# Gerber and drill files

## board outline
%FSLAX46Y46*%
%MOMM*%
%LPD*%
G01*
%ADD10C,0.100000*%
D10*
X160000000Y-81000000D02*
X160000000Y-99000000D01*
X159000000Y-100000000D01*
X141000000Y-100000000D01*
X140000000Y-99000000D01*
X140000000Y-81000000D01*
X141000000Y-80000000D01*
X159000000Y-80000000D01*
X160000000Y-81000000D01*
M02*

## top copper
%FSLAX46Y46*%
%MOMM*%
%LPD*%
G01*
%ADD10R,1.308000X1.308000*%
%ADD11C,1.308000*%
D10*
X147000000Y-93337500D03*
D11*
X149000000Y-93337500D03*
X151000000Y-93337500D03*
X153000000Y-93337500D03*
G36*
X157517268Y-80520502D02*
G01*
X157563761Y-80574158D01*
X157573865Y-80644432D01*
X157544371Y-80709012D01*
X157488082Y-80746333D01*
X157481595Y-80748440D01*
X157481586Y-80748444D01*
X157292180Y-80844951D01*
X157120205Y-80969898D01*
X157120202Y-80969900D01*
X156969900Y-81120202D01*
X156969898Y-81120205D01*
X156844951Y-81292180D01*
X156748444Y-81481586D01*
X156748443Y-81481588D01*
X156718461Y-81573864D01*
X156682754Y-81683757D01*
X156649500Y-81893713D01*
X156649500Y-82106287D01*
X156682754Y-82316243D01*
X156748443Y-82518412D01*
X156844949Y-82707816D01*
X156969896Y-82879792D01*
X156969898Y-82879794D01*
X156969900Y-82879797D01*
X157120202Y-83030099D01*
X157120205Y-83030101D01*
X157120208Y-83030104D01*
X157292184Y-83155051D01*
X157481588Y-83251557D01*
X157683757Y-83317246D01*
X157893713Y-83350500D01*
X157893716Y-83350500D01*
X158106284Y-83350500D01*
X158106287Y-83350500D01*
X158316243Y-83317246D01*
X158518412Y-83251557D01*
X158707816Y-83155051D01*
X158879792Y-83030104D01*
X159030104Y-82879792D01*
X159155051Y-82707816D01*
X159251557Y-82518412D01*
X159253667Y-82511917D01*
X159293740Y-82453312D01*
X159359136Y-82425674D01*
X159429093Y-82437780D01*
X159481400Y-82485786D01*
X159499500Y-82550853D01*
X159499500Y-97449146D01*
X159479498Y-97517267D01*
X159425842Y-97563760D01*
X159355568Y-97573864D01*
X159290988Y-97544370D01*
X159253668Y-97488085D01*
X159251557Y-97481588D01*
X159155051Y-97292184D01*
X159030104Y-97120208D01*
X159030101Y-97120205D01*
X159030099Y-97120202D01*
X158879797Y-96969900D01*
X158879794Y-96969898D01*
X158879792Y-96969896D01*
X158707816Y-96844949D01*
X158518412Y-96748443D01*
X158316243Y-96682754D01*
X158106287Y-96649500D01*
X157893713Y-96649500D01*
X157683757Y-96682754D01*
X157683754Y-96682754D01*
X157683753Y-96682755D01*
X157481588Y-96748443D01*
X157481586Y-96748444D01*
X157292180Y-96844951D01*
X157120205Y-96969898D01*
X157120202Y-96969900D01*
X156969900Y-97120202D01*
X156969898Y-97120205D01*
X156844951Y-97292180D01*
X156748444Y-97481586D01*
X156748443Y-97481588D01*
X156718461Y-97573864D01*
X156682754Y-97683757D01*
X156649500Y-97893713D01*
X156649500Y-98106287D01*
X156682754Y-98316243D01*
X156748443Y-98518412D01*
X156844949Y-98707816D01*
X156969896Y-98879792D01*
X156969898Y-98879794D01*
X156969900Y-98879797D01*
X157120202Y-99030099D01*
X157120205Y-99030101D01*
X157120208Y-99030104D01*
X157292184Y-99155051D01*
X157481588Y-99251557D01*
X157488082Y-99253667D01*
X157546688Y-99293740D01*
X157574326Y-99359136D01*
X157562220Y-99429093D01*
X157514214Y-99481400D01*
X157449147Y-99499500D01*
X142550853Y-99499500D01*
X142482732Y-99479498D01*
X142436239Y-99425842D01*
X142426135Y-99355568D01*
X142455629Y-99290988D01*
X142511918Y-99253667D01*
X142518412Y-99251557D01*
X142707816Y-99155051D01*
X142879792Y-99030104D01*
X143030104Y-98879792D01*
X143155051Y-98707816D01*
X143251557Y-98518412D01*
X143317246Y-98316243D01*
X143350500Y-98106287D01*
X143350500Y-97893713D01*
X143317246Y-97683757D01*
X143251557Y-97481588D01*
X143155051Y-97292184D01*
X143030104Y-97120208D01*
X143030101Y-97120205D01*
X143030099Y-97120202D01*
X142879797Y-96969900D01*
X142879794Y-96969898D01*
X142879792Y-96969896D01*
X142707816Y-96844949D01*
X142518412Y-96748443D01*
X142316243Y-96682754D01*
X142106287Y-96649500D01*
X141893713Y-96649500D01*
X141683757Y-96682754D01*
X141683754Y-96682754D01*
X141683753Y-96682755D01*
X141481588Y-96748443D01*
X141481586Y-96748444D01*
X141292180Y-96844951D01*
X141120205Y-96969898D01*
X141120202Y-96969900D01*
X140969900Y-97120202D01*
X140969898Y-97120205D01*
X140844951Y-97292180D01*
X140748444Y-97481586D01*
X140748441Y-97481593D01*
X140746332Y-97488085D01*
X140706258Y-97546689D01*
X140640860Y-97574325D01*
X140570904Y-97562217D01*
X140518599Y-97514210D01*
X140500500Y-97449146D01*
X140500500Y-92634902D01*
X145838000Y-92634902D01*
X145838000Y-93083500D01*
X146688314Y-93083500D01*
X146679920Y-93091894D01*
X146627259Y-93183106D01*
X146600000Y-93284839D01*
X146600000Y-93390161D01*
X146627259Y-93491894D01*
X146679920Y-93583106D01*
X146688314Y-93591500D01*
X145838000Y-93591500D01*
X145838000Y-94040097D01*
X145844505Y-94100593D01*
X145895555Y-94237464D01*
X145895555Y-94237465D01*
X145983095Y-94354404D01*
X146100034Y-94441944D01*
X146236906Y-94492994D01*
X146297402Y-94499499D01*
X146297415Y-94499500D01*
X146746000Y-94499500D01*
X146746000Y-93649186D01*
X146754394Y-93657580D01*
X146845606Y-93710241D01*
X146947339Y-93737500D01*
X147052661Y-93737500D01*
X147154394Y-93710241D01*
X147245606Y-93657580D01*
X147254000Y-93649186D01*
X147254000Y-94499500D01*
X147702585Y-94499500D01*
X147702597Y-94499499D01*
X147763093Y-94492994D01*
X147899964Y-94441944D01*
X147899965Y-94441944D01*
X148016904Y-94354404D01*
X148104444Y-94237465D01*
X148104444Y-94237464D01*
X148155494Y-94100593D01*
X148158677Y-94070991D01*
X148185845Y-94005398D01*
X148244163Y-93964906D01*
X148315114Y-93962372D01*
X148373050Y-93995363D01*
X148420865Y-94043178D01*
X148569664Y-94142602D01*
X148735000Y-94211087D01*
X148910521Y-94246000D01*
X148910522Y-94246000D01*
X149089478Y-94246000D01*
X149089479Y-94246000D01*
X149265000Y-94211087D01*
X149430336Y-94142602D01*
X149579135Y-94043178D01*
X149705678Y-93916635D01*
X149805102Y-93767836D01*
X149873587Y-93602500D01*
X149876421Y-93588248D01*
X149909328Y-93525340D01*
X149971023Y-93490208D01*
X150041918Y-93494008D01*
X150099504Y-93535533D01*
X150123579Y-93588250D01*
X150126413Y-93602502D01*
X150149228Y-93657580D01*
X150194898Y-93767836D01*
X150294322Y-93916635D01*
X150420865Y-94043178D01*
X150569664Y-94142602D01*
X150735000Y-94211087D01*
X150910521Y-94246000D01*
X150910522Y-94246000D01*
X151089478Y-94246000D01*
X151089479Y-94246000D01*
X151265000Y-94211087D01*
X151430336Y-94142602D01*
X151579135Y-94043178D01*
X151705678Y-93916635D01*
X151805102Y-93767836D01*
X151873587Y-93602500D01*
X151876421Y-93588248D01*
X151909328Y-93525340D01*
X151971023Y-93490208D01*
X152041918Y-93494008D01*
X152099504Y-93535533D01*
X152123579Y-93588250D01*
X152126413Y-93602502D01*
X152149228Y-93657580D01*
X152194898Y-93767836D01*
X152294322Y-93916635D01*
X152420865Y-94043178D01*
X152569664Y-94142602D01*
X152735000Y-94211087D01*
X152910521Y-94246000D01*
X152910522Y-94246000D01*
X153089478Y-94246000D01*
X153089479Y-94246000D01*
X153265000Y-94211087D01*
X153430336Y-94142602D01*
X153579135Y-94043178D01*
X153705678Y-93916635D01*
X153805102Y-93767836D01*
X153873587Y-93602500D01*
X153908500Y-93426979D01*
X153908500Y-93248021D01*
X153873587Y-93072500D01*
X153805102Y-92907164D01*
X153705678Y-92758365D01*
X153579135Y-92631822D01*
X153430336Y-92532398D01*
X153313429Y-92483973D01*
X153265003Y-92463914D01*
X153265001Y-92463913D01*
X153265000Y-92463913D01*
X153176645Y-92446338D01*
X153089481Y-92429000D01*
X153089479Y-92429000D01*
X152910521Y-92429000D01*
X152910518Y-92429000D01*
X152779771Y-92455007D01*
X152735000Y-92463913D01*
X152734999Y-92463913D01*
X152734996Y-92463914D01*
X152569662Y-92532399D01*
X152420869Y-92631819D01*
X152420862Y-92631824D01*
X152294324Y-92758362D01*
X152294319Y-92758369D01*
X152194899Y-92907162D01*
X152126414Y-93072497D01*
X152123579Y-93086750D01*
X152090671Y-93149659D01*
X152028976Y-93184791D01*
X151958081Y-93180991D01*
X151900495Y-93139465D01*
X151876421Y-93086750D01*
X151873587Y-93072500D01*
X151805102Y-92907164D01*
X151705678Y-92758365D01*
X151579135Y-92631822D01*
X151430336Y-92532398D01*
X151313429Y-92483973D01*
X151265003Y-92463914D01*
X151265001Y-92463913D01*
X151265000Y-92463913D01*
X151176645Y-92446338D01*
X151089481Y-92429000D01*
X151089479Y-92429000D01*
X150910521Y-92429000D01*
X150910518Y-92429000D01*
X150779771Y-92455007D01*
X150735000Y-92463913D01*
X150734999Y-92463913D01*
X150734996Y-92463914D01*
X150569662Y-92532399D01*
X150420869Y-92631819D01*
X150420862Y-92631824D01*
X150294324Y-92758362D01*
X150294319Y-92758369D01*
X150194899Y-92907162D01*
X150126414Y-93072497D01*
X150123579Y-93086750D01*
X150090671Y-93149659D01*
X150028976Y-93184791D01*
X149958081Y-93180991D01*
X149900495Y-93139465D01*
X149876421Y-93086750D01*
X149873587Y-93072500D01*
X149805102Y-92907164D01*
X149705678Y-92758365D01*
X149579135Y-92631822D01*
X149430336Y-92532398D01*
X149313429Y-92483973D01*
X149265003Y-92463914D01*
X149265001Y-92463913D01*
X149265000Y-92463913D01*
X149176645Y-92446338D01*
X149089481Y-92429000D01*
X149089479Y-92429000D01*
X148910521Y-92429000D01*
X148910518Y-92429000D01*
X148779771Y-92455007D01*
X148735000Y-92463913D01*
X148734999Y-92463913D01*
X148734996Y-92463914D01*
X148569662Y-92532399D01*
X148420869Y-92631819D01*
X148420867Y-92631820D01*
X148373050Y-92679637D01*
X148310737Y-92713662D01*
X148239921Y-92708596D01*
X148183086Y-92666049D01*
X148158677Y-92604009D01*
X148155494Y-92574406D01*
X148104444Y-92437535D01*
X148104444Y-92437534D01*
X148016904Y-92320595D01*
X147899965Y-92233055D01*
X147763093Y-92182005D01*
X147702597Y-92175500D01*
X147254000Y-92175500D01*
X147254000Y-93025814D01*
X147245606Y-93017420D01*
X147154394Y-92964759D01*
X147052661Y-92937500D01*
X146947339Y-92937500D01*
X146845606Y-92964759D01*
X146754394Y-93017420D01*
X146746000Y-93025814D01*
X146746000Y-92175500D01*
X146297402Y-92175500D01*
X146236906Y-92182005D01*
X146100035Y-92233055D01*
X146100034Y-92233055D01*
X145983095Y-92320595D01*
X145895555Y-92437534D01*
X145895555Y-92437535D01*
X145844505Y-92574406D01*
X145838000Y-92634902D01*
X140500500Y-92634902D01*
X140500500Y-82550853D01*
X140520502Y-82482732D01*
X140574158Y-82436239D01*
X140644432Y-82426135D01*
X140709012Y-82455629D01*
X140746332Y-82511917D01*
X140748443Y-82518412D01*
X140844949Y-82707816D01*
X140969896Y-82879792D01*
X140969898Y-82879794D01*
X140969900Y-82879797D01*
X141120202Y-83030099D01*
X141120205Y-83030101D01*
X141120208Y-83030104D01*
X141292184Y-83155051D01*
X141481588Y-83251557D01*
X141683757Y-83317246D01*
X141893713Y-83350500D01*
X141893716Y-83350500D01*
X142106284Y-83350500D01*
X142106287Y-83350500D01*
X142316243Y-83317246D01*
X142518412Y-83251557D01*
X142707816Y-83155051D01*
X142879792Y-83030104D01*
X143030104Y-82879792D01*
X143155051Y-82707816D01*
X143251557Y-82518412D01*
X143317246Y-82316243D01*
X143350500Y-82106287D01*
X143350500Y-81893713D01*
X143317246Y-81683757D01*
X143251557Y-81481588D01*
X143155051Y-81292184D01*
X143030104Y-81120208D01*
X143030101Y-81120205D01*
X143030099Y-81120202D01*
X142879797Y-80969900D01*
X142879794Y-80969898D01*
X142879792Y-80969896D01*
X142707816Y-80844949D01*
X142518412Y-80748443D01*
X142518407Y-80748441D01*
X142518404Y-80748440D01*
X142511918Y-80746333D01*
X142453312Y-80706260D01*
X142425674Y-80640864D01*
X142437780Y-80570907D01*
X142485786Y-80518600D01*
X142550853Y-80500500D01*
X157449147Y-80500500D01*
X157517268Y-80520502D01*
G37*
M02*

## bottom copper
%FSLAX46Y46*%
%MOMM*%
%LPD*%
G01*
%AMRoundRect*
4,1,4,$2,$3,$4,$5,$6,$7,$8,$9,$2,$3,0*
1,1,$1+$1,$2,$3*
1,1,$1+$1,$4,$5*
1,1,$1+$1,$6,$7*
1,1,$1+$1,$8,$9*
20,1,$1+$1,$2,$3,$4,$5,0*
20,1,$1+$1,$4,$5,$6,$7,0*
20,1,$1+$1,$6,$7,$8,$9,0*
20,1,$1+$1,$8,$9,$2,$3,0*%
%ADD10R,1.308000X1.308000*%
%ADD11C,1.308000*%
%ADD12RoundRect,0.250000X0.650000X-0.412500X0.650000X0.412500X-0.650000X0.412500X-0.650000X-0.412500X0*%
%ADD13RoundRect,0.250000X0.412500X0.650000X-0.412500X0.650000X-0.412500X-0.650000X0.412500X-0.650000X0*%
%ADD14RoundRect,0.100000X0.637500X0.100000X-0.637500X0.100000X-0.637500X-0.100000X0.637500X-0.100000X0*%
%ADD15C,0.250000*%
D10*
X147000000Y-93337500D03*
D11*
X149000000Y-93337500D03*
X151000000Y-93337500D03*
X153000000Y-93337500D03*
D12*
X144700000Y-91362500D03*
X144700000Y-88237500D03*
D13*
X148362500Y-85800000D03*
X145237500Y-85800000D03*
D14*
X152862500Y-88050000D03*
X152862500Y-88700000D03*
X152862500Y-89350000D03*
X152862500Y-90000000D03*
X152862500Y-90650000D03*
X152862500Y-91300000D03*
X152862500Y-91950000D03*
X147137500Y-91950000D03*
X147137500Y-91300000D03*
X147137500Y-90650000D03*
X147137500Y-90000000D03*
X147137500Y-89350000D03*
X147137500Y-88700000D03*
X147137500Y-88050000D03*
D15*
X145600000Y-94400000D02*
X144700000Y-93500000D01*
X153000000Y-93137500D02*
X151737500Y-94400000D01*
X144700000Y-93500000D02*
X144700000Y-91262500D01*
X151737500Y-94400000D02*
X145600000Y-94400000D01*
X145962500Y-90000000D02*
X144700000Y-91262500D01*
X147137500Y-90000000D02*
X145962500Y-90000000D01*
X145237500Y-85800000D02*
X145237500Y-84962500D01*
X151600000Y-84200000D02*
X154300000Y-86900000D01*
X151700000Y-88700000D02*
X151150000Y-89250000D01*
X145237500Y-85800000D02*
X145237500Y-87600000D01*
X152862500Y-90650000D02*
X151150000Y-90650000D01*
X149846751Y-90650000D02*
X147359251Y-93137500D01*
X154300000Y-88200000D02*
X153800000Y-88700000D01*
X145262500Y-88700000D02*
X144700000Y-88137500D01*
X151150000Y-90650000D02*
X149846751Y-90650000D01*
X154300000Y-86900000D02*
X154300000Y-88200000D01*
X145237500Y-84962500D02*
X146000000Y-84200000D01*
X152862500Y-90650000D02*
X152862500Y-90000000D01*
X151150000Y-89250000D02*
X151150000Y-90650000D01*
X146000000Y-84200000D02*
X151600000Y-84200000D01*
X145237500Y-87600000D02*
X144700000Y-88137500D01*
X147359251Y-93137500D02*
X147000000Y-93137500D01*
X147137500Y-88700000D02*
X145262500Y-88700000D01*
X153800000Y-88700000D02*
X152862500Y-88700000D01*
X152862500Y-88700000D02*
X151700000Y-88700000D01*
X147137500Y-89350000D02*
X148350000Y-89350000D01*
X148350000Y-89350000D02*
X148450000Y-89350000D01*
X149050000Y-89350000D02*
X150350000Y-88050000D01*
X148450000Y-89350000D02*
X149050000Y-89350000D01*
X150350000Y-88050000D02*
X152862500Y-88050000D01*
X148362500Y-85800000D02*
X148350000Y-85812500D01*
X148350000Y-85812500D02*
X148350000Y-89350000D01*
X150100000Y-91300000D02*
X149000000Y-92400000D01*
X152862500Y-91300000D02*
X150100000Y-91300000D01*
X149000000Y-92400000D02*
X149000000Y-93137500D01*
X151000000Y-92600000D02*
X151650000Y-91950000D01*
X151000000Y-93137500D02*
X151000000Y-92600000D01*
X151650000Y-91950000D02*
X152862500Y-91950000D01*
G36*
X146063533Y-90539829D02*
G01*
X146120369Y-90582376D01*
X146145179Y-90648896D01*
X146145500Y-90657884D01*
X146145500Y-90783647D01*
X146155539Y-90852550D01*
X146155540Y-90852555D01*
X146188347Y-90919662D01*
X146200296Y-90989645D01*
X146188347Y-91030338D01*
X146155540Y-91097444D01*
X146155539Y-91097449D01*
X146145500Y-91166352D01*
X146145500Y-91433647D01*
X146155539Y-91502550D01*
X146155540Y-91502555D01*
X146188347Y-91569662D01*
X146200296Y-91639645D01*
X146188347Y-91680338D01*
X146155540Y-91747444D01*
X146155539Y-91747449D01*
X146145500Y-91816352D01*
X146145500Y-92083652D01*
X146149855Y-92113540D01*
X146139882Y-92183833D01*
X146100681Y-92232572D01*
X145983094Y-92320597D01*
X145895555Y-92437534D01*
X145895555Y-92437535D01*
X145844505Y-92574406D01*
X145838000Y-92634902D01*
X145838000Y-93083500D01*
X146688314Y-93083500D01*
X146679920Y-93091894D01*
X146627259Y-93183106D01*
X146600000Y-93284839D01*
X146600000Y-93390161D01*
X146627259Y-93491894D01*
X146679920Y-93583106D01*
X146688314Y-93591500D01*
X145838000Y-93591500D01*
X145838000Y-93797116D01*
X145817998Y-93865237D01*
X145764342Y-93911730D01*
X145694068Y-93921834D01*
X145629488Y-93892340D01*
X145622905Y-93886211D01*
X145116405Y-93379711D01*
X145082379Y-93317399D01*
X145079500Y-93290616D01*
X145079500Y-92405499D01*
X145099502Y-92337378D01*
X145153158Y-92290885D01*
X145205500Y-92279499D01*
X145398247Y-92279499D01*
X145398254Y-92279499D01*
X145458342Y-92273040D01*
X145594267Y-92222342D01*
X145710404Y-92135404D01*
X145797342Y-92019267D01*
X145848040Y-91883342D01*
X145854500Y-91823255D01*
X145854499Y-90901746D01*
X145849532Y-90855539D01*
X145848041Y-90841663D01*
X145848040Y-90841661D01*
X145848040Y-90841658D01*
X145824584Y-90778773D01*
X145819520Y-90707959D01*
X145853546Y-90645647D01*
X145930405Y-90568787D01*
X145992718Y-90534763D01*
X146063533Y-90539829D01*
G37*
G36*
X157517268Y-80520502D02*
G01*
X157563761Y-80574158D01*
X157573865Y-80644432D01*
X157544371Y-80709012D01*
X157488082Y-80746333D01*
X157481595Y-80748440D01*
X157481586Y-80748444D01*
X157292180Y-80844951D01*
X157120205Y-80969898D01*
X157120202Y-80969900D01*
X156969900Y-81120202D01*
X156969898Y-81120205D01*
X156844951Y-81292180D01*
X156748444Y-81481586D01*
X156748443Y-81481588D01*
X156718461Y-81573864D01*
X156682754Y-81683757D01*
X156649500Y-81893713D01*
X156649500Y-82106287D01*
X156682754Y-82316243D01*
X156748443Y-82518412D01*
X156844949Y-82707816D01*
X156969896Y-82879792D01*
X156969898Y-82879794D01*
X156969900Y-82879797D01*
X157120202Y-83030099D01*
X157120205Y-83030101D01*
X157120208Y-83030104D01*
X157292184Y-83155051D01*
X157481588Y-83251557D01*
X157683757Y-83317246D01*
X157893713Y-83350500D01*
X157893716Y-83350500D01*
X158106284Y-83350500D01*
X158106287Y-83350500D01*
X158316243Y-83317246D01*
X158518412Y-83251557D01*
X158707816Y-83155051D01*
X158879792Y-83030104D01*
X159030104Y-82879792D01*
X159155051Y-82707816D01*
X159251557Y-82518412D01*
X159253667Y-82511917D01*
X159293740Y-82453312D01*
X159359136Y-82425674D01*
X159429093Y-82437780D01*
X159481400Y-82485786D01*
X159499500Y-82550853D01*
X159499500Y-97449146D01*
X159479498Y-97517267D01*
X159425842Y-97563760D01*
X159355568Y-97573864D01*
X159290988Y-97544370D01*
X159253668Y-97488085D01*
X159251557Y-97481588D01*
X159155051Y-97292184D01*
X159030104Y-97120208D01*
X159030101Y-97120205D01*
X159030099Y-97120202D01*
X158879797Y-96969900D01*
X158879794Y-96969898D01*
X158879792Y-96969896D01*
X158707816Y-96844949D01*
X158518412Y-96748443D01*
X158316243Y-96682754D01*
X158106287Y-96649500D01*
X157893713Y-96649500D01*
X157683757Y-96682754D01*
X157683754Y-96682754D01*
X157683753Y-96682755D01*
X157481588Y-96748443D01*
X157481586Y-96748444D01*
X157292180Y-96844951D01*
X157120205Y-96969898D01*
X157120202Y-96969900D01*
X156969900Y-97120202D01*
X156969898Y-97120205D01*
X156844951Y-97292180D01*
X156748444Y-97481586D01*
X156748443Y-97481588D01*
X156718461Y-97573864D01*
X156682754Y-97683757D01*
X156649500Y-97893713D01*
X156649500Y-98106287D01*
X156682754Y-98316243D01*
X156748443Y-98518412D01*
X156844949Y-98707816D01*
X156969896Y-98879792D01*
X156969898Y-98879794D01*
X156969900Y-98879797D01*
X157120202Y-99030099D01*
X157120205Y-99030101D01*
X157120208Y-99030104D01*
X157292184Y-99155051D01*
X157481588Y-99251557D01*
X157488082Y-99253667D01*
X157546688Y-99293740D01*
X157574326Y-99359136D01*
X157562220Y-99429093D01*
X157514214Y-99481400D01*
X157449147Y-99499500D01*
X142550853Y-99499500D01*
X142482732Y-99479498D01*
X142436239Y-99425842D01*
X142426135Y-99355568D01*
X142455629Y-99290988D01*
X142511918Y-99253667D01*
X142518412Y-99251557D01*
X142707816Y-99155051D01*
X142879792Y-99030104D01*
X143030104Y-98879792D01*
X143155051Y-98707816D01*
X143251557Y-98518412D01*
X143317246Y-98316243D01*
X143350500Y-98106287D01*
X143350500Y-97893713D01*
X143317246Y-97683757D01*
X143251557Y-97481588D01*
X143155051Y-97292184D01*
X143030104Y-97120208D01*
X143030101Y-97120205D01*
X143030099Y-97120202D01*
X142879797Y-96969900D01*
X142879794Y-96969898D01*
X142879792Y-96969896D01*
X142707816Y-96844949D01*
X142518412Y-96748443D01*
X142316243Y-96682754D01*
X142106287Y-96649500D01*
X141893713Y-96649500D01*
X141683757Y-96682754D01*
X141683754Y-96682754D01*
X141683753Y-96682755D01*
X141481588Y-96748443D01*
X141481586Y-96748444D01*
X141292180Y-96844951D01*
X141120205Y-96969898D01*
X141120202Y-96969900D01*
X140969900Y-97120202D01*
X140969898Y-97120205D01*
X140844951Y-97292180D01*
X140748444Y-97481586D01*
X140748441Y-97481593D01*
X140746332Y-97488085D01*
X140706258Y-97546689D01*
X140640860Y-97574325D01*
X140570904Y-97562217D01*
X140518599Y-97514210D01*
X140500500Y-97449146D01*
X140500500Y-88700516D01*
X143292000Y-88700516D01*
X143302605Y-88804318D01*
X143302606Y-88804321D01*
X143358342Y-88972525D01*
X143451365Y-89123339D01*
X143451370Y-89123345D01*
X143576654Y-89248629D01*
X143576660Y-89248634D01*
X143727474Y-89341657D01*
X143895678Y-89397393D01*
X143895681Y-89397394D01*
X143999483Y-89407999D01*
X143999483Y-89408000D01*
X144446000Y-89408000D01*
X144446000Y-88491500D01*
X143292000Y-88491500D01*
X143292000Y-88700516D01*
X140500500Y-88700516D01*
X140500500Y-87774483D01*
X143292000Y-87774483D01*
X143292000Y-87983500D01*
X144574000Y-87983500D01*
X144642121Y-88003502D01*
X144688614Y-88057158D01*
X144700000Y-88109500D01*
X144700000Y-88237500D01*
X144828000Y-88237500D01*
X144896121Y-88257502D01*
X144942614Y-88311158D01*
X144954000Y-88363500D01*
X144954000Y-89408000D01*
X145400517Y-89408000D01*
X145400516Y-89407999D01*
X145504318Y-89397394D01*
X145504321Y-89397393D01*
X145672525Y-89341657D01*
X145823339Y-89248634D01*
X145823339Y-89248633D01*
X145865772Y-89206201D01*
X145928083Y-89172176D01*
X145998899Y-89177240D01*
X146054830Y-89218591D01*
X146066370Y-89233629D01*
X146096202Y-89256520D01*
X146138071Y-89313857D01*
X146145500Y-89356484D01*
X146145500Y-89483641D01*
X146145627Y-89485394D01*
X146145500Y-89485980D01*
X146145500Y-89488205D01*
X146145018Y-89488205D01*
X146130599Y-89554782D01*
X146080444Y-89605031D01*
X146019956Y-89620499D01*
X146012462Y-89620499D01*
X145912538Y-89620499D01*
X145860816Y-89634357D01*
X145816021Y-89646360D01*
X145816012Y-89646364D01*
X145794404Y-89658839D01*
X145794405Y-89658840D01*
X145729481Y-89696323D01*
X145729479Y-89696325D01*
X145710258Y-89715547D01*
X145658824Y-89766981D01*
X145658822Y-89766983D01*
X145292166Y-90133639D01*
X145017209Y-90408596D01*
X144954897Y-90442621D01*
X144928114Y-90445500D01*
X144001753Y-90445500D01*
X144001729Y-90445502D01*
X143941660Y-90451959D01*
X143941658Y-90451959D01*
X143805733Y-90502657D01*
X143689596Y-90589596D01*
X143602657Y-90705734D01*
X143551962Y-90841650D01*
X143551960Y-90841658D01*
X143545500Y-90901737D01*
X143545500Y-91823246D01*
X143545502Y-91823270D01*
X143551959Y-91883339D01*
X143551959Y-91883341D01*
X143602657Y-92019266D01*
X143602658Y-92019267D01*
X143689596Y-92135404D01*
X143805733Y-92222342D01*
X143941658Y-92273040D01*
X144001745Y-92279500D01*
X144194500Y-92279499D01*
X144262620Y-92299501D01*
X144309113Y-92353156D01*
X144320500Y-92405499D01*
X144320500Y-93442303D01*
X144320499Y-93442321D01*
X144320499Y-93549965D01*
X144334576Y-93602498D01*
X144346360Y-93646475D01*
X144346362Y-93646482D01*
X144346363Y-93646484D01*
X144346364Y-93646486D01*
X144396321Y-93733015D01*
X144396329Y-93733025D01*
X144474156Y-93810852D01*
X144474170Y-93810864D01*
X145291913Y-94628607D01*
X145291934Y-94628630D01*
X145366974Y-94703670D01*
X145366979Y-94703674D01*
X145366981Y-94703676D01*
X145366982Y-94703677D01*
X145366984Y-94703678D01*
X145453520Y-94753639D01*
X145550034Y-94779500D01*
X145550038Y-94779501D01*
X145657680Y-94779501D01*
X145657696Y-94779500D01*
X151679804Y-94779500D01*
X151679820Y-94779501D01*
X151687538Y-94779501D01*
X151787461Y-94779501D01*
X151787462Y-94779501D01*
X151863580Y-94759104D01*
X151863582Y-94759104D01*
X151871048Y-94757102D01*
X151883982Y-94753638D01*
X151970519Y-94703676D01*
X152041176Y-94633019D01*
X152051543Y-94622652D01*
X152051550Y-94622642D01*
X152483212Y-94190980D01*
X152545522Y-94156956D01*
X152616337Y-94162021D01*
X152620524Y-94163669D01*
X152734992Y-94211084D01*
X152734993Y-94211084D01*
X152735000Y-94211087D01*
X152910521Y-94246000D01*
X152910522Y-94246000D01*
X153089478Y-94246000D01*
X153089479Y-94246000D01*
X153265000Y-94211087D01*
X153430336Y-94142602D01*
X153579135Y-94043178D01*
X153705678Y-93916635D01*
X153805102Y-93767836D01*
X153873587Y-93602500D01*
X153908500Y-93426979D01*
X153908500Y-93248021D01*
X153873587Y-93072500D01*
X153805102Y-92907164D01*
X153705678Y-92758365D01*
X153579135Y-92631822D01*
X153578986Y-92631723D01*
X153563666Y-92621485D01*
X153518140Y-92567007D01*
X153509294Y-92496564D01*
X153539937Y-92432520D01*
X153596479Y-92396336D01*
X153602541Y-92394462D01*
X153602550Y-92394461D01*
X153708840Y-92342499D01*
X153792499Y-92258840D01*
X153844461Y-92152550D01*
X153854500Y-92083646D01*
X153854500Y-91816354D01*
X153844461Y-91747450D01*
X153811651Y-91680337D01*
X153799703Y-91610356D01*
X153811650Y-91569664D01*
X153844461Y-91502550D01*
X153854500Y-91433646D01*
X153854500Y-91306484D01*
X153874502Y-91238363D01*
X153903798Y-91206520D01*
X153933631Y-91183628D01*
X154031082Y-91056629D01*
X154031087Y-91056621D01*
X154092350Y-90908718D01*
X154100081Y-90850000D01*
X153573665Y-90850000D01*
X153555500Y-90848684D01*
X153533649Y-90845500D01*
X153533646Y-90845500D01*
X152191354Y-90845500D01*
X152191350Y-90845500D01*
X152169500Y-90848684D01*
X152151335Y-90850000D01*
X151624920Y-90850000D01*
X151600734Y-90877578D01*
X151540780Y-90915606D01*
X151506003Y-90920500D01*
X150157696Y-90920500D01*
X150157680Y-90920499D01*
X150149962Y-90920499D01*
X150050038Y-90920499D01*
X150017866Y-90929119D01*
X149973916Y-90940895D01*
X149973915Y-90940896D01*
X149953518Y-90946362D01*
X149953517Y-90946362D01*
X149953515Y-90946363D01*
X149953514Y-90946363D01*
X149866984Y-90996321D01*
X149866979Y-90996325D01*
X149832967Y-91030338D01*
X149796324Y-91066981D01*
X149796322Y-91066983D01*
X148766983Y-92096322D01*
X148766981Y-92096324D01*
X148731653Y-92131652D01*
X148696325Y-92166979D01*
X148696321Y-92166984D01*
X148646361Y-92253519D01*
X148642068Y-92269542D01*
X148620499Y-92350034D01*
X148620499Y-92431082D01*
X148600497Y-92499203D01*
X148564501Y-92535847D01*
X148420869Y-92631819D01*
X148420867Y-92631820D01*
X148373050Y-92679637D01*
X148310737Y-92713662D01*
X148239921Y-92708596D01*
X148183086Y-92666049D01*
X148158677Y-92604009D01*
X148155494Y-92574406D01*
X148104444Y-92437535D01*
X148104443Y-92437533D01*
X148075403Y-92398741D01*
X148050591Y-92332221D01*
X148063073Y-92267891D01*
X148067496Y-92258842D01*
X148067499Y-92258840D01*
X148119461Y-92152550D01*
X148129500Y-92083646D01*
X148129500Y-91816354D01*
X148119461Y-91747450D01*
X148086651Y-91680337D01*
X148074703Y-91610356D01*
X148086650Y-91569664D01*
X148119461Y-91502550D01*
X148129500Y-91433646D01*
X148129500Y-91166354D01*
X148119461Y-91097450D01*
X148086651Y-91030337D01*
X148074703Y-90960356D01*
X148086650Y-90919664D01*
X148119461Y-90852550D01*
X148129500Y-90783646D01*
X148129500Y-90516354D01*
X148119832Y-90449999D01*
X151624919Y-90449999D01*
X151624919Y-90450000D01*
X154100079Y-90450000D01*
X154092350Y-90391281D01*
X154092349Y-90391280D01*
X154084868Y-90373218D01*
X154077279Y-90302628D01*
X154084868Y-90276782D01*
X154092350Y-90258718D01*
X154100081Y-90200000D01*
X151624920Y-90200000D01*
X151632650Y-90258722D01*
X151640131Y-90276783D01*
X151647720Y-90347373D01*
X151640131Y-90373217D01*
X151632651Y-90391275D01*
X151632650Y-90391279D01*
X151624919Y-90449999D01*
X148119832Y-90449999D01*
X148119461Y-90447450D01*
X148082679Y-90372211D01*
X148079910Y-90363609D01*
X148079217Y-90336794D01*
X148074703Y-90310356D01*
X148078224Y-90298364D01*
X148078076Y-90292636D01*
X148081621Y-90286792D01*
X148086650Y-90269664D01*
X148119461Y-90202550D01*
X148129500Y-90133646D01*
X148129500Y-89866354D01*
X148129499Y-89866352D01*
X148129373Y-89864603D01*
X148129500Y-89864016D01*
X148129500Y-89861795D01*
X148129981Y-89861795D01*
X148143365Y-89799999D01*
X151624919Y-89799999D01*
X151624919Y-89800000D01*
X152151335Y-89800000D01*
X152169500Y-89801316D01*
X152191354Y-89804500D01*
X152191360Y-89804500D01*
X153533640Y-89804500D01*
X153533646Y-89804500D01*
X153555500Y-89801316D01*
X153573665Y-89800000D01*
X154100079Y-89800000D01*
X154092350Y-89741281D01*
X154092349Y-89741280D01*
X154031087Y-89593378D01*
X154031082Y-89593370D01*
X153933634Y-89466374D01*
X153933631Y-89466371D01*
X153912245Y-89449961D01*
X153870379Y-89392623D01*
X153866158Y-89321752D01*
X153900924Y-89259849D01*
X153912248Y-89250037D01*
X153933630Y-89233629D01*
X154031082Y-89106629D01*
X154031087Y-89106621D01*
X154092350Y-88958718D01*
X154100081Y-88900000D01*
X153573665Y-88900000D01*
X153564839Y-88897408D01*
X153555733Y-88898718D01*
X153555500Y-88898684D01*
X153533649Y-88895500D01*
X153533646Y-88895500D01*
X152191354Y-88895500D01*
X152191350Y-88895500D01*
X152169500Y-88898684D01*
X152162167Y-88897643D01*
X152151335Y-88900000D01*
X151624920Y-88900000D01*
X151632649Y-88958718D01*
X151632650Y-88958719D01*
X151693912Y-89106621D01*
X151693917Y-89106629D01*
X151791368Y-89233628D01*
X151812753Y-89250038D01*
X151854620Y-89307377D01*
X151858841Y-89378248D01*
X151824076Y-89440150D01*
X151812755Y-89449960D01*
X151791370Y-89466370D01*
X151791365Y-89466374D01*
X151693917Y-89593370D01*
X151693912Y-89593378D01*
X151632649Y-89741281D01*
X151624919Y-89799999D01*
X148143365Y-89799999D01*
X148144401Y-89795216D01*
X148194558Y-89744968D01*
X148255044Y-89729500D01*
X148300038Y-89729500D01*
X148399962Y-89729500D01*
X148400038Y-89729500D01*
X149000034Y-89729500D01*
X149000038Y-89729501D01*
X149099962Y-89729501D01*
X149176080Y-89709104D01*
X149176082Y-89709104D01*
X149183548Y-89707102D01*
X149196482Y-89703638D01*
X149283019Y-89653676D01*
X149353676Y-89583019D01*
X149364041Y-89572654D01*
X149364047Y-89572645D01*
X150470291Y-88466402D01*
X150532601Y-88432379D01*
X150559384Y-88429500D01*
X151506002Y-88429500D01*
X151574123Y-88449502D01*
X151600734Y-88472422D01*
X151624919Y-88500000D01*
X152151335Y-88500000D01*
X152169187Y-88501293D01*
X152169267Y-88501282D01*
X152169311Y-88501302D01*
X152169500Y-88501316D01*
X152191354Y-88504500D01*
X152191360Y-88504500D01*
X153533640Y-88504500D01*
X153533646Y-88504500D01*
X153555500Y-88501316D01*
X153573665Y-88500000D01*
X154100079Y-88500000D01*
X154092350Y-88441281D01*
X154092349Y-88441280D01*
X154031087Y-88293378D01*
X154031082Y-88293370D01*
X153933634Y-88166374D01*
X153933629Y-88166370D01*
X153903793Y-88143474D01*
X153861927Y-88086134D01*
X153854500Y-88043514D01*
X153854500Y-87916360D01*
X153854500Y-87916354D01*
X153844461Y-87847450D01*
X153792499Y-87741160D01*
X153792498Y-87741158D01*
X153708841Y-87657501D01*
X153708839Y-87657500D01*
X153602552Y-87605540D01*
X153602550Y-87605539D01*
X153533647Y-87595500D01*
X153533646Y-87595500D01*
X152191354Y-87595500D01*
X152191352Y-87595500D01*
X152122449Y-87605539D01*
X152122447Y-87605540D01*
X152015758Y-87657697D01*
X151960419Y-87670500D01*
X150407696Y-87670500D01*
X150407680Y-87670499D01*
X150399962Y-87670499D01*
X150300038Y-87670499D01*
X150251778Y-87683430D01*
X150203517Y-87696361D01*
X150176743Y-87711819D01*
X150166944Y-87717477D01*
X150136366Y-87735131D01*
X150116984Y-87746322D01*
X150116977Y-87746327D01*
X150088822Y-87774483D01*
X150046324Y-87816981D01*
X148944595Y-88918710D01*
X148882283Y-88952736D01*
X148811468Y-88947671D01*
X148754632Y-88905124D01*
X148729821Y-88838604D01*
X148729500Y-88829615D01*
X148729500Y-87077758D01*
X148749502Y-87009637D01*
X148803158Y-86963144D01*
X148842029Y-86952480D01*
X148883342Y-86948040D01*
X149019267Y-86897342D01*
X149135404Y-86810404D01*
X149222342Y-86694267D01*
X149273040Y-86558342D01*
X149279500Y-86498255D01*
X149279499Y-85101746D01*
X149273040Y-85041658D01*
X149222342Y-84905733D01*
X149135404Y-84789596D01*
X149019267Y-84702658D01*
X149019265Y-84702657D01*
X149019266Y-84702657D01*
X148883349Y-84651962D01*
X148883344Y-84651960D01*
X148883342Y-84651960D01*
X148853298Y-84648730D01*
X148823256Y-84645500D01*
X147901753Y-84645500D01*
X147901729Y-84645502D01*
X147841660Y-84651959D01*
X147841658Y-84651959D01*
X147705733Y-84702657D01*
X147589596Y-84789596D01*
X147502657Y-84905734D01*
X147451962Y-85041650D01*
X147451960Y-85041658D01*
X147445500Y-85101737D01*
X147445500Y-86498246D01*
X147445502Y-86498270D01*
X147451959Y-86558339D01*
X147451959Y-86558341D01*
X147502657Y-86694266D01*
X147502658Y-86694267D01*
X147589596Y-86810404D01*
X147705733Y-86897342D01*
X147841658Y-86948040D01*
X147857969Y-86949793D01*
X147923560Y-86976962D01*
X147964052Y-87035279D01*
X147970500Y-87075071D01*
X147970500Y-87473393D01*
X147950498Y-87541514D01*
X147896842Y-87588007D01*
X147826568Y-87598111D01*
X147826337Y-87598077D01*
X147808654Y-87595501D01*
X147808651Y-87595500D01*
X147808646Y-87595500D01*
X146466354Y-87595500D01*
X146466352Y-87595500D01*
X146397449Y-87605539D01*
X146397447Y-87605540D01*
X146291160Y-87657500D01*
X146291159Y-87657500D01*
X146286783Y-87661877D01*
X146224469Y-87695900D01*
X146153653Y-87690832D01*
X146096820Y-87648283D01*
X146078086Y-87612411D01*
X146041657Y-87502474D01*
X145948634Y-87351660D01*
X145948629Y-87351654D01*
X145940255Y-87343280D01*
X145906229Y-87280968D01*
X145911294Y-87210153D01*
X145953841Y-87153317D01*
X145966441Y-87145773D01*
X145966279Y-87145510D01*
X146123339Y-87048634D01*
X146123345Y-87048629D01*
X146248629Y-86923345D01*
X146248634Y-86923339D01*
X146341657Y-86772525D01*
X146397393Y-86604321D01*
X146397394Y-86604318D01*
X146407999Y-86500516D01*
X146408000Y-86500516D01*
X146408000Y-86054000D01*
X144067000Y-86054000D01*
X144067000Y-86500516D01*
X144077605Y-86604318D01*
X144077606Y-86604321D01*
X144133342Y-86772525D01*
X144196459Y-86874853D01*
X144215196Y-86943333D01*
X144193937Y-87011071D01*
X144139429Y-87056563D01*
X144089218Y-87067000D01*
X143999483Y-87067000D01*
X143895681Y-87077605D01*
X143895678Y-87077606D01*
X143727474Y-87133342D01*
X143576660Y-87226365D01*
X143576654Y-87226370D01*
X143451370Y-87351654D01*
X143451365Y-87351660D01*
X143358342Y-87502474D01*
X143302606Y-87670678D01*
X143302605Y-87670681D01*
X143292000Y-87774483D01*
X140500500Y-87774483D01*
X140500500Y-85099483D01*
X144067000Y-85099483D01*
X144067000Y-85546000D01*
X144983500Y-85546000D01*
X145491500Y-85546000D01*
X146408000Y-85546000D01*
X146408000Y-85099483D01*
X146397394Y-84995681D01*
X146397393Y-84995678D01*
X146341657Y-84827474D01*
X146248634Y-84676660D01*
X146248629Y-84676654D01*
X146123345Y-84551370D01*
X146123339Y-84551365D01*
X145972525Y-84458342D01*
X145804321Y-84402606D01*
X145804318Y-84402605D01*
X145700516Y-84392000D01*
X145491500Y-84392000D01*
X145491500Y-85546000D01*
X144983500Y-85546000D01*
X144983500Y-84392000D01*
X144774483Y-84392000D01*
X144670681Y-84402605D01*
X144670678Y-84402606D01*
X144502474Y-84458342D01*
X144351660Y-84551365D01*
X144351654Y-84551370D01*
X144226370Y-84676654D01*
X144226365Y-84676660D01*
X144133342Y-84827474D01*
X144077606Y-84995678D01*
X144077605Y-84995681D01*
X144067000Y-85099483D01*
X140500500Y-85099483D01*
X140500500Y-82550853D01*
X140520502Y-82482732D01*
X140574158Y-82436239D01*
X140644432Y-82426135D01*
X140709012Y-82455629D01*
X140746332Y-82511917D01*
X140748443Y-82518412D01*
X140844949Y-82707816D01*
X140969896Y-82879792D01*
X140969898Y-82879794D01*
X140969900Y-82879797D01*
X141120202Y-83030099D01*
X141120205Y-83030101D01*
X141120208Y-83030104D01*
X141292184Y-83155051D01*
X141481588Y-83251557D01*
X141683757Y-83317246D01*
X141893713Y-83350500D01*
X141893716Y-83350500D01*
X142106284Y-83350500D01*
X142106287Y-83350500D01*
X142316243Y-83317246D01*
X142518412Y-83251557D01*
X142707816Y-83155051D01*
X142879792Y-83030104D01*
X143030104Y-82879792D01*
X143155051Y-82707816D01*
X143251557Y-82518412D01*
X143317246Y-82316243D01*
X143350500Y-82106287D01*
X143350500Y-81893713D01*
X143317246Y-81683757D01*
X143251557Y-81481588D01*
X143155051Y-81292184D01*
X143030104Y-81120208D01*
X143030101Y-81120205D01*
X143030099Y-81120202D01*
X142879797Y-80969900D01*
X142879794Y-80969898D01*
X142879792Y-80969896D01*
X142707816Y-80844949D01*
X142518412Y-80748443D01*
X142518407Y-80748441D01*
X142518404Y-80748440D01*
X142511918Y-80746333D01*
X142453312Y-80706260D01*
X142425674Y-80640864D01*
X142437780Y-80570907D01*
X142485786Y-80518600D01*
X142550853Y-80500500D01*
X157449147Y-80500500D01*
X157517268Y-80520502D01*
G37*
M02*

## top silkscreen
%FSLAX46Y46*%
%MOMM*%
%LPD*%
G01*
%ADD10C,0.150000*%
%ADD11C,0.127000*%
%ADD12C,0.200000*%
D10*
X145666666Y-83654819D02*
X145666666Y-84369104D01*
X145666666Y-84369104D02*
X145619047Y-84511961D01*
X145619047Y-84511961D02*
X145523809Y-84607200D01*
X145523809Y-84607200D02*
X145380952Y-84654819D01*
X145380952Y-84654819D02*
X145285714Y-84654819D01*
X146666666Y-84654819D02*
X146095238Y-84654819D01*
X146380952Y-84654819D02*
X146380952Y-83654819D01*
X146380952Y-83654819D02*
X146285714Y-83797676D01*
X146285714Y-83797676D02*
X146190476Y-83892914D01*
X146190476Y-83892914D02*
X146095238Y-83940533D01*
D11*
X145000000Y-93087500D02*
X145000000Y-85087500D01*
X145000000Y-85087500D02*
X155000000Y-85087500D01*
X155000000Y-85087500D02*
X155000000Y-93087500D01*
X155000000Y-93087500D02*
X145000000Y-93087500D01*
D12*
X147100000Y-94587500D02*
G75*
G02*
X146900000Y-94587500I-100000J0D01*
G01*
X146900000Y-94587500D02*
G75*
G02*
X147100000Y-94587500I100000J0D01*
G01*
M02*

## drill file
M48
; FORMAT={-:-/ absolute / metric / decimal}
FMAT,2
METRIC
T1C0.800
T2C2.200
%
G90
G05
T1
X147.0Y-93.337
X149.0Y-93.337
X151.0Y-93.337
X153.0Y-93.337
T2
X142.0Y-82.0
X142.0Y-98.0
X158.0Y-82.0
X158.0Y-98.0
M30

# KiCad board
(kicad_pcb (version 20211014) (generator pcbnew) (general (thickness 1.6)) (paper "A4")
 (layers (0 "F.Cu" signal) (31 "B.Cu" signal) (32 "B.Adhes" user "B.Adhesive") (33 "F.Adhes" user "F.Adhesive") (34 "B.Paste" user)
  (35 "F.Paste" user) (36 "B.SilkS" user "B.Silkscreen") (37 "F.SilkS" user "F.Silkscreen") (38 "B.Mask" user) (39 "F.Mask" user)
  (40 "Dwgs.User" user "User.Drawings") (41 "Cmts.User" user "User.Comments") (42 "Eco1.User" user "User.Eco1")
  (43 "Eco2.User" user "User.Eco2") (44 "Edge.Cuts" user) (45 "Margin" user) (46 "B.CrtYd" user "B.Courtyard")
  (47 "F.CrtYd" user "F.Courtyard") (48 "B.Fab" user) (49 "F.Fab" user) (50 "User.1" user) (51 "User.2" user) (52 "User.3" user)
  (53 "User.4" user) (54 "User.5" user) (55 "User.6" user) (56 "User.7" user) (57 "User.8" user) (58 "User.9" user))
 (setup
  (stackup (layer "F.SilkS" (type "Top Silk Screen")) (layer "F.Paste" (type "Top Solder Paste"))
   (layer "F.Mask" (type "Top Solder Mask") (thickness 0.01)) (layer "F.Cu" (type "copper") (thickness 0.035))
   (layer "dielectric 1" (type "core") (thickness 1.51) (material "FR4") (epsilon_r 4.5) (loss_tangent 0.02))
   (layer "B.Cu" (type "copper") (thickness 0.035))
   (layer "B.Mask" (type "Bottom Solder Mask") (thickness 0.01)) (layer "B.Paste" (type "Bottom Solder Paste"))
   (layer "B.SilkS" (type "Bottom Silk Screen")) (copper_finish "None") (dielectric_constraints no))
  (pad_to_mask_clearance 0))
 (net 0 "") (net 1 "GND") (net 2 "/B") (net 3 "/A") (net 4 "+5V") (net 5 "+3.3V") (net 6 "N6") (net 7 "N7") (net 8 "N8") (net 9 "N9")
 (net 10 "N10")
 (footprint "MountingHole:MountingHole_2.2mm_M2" (layer "F.Cu") (at 142 82)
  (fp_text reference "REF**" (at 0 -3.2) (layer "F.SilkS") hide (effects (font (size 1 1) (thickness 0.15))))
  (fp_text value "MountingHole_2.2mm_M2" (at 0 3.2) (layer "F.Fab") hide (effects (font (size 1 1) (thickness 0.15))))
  (pad "" np_thru_hole circle (at 0 0) (size 2.2 2.2) (drill 2.2) (layers F&B.Cu *.Mask)))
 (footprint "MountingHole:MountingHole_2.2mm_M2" (layer "F.Cu") (at 158 98)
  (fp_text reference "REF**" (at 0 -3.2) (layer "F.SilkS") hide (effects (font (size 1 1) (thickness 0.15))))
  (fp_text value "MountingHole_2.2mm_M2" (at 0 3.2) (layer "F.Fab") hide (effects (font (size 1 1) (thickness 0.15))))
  (pad "" np_thru_hole circle (at 0 0) (size 2.2 2.2) (drill 2.2) (layers F&B.Cu *.Mask)))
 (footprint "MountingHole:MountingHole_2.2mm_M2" (layer "F.Cu") (at 142 98)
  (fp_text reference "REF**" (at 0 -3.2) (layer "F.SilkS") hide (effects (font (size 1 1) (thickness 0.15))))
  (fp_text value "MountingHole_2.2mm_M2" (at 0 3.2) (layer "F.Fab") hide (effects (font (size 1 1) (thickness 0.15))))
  (pad "" np_thru_hole circle (at 0 0) (size 2.2 2.2) (drill 2.2) (layers *.Cu *.Mask)))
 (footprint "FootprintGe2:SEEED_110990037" (layer "F.Cu") (at 150 93.3375)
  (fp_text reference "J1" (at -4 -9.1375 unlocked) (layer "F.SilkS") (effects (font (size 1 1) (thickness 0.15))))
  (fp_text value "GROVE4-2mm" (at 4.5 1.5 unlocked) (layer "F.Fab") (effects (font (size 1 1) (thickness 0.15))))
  (fp_line (start -5 -0.25) (end -5 -8.25) (layer "F.SilkS") (width 0.127))
  (fp_line (start -5 -8.25) (end 5 -8.25) (layer "F.SilkS") (width 0.127))
  (fp_line (start 5 -8.25) (end 5 -0.25) (layer "F.SilkS") (width 0.127))
  (fp_line (start 5 -0.25) (end -5 -0.25) (layer "F.SilkS") (width 0.127))
  (fp_circle (center -3 1.25) (end -2.9 1.25) (layer "F.SilkS") (width 0.2) (fill none))
  (pad "1" thru_hole rect (at -3 0) (size 1.308 1.308) (drill 0.8) (layers *.Cu *.Mask) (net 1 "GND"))
  (pad "2" thru_hole circle (at -1 0) (size 1.308 1.308) (drill 0.8) (layers *.Cu *.Mask) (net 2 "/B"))
  (pad "3" thru_hole circle (at 1 0) (size 1.308 1.308) (drill 0.8) (layers *.Cu *.Mask) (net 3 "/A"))
  (pad "4" thru_hole circle (at 3 0) (size 1.308 1.308) (drill 0.8) (layers *.Cu *.Mask) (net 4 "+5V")))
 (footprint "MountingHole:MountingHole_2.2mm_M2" (layer "F.Cu") (at 158 82)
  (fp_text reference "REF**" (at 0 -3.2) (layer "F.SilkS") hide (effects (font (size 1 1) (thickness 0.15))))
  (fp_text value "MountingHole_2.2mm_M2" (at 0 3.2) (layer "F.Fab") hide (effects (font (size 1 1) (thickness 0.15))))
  (pad "" np_thru_hole circle (at 0 0) (size 2.2 2.2) (drill 2.2) (layers F&B.Cu *.Mask)))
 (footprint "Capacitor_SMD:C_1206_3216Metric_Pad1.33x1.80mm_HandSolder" (layer "B.Cu") (at 144.7 89.8 90)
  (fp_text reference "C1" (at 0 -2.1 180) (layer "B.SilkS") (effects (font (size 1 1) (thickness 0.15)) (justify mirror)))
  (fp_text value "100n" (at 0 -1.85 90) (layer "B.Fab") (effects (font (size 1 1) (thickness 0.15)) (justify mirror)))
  (pad "1" smd roundrect (at -1.5625 0 90) (size 1.325 1.8) (layers "B.Cu" "B.Paste" "B.Mask") (roundrect_rratio 0.1886792453) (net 4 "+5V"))
  (pad "2" smd roundrect (at 1.5625 0 90) (size 1.325 1.8) (layers "B.Cu" "B.Paste" "B.Mask") (roundrect_rratio 0.1886792453) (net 1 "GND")))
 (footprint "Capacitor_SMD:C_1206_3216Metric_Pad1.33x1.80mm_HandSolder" (layer "B.Cu") (at 146.8 85.8 180)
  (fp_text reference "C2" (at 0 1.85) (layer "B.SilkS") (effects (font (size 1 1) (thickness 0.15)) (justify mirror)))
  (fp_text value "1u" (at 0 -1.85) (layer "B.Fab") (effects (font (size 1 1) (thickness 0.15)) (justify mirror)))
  (pad "1" smd roundrect (at -1.5625 0 180) (size 1.325 1.8) (layers "B.Cu" "B.Paste" "B.Mask") (roundrect_rratio 0.1886792453)
   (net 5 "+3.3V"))
  (pad "2" smd roundrect (at 1.5625 0 180) (size 1.325 1.8) (layers "B.Cu" "B.Paste" "B.Mask") (roundrect_rratio 0.1886792453) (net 1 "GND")))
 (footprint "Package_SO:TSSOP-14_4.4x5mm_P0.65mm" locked (layer "B.Cu") (at 150 90 180)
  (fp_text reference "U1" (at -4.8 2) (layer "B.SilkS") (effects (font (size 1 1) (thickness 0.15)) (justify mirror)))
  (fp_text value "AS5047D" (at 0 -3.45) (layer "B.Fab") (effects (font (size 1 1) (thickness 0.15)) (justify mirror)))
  (pad "1" smd roundrect locked (at -2.8625 1.95 180) (size 1.475 0.4) (layers "B.Cu" "B.Paste" "B.Mask") (roundrect_rratio 0.25)
   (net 5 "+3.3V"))
  (pad "2" smd roundrect locked (at -2.8625 1.3 180) (size 1.475 0.4) (layers "B.Cu" "B.Paste" "B.Mask") (roundrect_rratio 0.25)
   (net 1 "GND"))
  (pad "3" smd roundrect locked (at -2.8625 0.65 180) (size 1.475 0.4) (layers "B.Cu" "B.Paste" "B.Mask") (roundrect_rratio 0.25)
   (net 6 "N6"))
  (pad "4" smd roundrect locked (at -2.8625 0 180) (size 1.475 0.4) (layers "B.Cu" "B.Paste" "B.Mask") (roundrect_rratio 0.25) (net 1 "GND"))
  (pad "5" smd roundrect locked (at -2.8625 -0.65 180) (size 1.475 0.4) (layers "B.Cu" "B.Paste" "B.Mask") (roundrect_rratio 0.25)
   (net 1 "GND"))
  (pad "6" smd roundrect locked (at -2.8625 -1.3 180) (size 1.475 0.4) (layers "B.Cu" "B.Paste" "B.Mask") (roundrect_rratio 0.25)
   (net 2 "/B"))
  (pad "7" smd roundrect locked (at -2.8625 -1.95 180) (size 1.475 0.4) (layers "B.Cu" "B.Paste" "B.Mask") (roundrect_rratio 0.25)
   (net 3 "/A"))
  (pad "8" smd roundrect locked (at 2.8625 -1.95 180) (size 1.475 0.4) (layers "B.Cu" "B.Paste" "B.Mask") (roundrect_rratio 0.25)
   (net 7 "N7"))
  (pad "9" smd roundrect locked (at 2.8625 -1.3 180) (size 1.475 0.4) (layers "B.Cu" "B.Paste" "B.Mask") (roundrect_rratio 0.25)
   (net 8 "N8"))
  (pad "10" smd roundrect locked (at 2.8625 -0.65 180) (size 1.475 0.4) (layers "B.Cu" "B.Paste" "B.Mask") (roundrect_rratio 0.25)
   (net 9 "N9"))
  (pad "11" smd roundrect locked (at 2.8625 0 180) (size 1.475 0.4) (layers "B.Cu" "B.Paste" "B.Mask") (roundrect_rratio 0.25) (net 4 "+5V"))
  (pad "12" smd roundrect locked (at 2.8625 0.65 180) (size 1.475 0.4) (layers "B.Cu" "B.Paste" "B.Mask") (roundrect_rratio 0.25)
   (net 5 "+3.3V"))
  (pad "13" smd roundrect locked (at 2.8625 1.3 180) (size 1.475 0.4) (layers "B.Cu" "B.Paste" "B.Mask") (roundrect_rratio 0.25)
   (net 1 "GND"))
  (pad "14" smd roundrect locked (at 2.8625 1.95 180) (size 1.475 0.4) (layers "B.Cu" "B.Paste" "B.Mask") (roundrect_rratio 0.25)
   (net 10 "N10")))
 (gr_poly
  (pts (xy 160 81) (xy 160 99) (xy 159 100) (xy 141 100) (xy 140 99) (xy 140 81) (xy 141 80) (xy 159 80)) (layer "Edge.Cuts") (width 0.1)
  (fill none))
 (segment (start 145.6 94.4) (end 144.7 93.5) (width 0.25) (layer "B.Cu") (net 4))
 (segment (start 153 93.1375) (end 151.7375 94.4) (width 0.25) (layer "B.Cu") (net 4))
 (segment (start 144.7 93.5) (end 144.7 91.2625) (width 0.25) (layer "B.Cu") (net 4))
 (segment (start 151.7375 94.4) (end 145.6 94.4) (width 0.25) (layer "B.Cu") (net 4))
 (segment (start 145.9625 90) (end 144.7 91.2625) (width 0.25) (layer "B.Cu") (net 4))
 (segment (start 147.1375 90) (end 145.9625 90) (width 0.25) (layer "B.Cu") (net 4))
 (segment (start 145.2375 85.8) (end 145.2375 84.9625) (width 0.25) (layer "B.Cu") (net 1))
 (segment (start 151.6 84.2) (end 154.3 86.9) (width 0.25) (layer "B.Cu") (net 1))
 (segment (start 151.7 88.7) (end 151.15 89.25) (width 0.25) (layer "B.Cu") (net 1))
 (segment (start 145.2375 85.8) (end 145.2375 87.6) (width 0.25) (layer "B.Cu") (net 1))
 (segment (start 152.8625 90.65) (end 151.15 90.65) (width 0.25) (layer "B.Cu") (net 1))
 (segment (start 149.846751 90.65) (end 147.359251 93.1375) (width 0.25) (layer "B.Cu") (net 1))
 (segment (start 154.3 88.2) (end 153.8 88.7) (width 0.25) (layer "B.Cu") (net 1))
 (segment (start 145.2625 88.7) (end 144.7 88.1375) (width 0.25) (layer "B.Cu") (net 1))
 (segment (start 151.15 90.65) (end 149.846751 90.65) (width 0.25) (layer "B.Cu") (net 1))
 (segment (start 154.3 86.9) (end 154.3 88.2) (width 0.25) (layer "B.Cu") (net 1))
 (segment (start 145.2375 84.9625) (end 146 84.2) (width 0.25) (layer "B.Cu") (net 1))
 (segment (start 152.8625 90.65) (end 152.8625 90) (width 0.25) (layer "B.Cu") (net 1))
 (segment (start 151.15 89.25) (end 151.15 90.65) (width 0.25) (layer "B.Cu") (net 1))
 (segment (start 146 84.2) (end 151.6 84.2) (width 0.25) (layer "B.Cu") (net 1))
 (segment (start 145.2375 87.6) (end 144.7 88.1375) (width 0.25) (layer "B.Cu") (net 1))
 (segment (start 147.359251 93.1375) (end 147 93.1375) (width 0.25) (layer "B.Cu") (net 1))
 (segment (start 147.1375 88.7) (end 145.2625 88.7) (width 0.25) (layer "B.Cu") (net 1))
 (segment (start 153.8 88.7) (end 152.8625 88.7) (width 0.25) (layer "B.Cu") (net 1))
 (segment (start 152.8625 88.7) (end 151.7 88.7) (width 0.25) (layer "B.Cu") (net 1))
 (segment (start 147.1375 89.35) (end 148.35 89.35) (width 0.25) (layer "B.Cu") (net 5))
 (segment (start 148.35 89.35) (end 148.45 89.35) (width 0.25) (layer "B.Cu") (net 5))
 (segment (start 149.05 89.35) (end 150.35 88.05) (width 0.25) (layer "B.Cu") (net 5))
 (segment (start 148.45 89.35) (end 149.05 89.35) (width 0.25) (layer "B.Cu") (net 5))
 (segment (start 150.35 88.05) (end 152.8625 88.05) (width 0.25) (layer "B.Cu") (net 5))
 (segment (start 148.3625 85.8) (end 148.35 85.8125) (width 0.25) (layer "B.Cu") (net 5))
 (segment (start 148.35 85.8125) (end 148.35 89.35) (width 0.25) (layer "B.Cu") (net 5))
 (segment (start 150.1 91.3) (end 149 92.4) (width 0.25) (layer "B.Cu") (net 2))
 (segment (start 152.8625 91.3) (end 150.1 91.3) (width 0.25) (layer "B.Cu") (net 2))
 (segment (start 149 92.4) (end 149 93.1375) (width 0.25) (layer "B.Cu") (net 2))
 (segment (start 151 92.6) (end 151.65 91.95) (width 0.25) (layer "B.Cu") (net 3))
 (segment (start 151 93.1375) (end 151 92.6) (width 0.25) (layer "B.Cu") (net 3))
 (segment (start 151.65 91.95) (end 152.8625 91.95) (width 0.25) (layer "B.Cu") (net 3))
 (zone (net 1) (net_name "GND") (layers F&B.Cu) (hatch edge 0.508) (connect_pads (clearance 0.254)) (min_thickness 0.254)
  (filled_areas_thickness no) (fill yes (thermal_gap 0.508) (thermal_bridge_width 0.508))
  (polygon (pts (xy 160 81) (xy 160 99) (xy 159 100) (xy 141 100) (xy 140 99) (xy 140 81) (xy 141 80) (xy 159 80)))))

